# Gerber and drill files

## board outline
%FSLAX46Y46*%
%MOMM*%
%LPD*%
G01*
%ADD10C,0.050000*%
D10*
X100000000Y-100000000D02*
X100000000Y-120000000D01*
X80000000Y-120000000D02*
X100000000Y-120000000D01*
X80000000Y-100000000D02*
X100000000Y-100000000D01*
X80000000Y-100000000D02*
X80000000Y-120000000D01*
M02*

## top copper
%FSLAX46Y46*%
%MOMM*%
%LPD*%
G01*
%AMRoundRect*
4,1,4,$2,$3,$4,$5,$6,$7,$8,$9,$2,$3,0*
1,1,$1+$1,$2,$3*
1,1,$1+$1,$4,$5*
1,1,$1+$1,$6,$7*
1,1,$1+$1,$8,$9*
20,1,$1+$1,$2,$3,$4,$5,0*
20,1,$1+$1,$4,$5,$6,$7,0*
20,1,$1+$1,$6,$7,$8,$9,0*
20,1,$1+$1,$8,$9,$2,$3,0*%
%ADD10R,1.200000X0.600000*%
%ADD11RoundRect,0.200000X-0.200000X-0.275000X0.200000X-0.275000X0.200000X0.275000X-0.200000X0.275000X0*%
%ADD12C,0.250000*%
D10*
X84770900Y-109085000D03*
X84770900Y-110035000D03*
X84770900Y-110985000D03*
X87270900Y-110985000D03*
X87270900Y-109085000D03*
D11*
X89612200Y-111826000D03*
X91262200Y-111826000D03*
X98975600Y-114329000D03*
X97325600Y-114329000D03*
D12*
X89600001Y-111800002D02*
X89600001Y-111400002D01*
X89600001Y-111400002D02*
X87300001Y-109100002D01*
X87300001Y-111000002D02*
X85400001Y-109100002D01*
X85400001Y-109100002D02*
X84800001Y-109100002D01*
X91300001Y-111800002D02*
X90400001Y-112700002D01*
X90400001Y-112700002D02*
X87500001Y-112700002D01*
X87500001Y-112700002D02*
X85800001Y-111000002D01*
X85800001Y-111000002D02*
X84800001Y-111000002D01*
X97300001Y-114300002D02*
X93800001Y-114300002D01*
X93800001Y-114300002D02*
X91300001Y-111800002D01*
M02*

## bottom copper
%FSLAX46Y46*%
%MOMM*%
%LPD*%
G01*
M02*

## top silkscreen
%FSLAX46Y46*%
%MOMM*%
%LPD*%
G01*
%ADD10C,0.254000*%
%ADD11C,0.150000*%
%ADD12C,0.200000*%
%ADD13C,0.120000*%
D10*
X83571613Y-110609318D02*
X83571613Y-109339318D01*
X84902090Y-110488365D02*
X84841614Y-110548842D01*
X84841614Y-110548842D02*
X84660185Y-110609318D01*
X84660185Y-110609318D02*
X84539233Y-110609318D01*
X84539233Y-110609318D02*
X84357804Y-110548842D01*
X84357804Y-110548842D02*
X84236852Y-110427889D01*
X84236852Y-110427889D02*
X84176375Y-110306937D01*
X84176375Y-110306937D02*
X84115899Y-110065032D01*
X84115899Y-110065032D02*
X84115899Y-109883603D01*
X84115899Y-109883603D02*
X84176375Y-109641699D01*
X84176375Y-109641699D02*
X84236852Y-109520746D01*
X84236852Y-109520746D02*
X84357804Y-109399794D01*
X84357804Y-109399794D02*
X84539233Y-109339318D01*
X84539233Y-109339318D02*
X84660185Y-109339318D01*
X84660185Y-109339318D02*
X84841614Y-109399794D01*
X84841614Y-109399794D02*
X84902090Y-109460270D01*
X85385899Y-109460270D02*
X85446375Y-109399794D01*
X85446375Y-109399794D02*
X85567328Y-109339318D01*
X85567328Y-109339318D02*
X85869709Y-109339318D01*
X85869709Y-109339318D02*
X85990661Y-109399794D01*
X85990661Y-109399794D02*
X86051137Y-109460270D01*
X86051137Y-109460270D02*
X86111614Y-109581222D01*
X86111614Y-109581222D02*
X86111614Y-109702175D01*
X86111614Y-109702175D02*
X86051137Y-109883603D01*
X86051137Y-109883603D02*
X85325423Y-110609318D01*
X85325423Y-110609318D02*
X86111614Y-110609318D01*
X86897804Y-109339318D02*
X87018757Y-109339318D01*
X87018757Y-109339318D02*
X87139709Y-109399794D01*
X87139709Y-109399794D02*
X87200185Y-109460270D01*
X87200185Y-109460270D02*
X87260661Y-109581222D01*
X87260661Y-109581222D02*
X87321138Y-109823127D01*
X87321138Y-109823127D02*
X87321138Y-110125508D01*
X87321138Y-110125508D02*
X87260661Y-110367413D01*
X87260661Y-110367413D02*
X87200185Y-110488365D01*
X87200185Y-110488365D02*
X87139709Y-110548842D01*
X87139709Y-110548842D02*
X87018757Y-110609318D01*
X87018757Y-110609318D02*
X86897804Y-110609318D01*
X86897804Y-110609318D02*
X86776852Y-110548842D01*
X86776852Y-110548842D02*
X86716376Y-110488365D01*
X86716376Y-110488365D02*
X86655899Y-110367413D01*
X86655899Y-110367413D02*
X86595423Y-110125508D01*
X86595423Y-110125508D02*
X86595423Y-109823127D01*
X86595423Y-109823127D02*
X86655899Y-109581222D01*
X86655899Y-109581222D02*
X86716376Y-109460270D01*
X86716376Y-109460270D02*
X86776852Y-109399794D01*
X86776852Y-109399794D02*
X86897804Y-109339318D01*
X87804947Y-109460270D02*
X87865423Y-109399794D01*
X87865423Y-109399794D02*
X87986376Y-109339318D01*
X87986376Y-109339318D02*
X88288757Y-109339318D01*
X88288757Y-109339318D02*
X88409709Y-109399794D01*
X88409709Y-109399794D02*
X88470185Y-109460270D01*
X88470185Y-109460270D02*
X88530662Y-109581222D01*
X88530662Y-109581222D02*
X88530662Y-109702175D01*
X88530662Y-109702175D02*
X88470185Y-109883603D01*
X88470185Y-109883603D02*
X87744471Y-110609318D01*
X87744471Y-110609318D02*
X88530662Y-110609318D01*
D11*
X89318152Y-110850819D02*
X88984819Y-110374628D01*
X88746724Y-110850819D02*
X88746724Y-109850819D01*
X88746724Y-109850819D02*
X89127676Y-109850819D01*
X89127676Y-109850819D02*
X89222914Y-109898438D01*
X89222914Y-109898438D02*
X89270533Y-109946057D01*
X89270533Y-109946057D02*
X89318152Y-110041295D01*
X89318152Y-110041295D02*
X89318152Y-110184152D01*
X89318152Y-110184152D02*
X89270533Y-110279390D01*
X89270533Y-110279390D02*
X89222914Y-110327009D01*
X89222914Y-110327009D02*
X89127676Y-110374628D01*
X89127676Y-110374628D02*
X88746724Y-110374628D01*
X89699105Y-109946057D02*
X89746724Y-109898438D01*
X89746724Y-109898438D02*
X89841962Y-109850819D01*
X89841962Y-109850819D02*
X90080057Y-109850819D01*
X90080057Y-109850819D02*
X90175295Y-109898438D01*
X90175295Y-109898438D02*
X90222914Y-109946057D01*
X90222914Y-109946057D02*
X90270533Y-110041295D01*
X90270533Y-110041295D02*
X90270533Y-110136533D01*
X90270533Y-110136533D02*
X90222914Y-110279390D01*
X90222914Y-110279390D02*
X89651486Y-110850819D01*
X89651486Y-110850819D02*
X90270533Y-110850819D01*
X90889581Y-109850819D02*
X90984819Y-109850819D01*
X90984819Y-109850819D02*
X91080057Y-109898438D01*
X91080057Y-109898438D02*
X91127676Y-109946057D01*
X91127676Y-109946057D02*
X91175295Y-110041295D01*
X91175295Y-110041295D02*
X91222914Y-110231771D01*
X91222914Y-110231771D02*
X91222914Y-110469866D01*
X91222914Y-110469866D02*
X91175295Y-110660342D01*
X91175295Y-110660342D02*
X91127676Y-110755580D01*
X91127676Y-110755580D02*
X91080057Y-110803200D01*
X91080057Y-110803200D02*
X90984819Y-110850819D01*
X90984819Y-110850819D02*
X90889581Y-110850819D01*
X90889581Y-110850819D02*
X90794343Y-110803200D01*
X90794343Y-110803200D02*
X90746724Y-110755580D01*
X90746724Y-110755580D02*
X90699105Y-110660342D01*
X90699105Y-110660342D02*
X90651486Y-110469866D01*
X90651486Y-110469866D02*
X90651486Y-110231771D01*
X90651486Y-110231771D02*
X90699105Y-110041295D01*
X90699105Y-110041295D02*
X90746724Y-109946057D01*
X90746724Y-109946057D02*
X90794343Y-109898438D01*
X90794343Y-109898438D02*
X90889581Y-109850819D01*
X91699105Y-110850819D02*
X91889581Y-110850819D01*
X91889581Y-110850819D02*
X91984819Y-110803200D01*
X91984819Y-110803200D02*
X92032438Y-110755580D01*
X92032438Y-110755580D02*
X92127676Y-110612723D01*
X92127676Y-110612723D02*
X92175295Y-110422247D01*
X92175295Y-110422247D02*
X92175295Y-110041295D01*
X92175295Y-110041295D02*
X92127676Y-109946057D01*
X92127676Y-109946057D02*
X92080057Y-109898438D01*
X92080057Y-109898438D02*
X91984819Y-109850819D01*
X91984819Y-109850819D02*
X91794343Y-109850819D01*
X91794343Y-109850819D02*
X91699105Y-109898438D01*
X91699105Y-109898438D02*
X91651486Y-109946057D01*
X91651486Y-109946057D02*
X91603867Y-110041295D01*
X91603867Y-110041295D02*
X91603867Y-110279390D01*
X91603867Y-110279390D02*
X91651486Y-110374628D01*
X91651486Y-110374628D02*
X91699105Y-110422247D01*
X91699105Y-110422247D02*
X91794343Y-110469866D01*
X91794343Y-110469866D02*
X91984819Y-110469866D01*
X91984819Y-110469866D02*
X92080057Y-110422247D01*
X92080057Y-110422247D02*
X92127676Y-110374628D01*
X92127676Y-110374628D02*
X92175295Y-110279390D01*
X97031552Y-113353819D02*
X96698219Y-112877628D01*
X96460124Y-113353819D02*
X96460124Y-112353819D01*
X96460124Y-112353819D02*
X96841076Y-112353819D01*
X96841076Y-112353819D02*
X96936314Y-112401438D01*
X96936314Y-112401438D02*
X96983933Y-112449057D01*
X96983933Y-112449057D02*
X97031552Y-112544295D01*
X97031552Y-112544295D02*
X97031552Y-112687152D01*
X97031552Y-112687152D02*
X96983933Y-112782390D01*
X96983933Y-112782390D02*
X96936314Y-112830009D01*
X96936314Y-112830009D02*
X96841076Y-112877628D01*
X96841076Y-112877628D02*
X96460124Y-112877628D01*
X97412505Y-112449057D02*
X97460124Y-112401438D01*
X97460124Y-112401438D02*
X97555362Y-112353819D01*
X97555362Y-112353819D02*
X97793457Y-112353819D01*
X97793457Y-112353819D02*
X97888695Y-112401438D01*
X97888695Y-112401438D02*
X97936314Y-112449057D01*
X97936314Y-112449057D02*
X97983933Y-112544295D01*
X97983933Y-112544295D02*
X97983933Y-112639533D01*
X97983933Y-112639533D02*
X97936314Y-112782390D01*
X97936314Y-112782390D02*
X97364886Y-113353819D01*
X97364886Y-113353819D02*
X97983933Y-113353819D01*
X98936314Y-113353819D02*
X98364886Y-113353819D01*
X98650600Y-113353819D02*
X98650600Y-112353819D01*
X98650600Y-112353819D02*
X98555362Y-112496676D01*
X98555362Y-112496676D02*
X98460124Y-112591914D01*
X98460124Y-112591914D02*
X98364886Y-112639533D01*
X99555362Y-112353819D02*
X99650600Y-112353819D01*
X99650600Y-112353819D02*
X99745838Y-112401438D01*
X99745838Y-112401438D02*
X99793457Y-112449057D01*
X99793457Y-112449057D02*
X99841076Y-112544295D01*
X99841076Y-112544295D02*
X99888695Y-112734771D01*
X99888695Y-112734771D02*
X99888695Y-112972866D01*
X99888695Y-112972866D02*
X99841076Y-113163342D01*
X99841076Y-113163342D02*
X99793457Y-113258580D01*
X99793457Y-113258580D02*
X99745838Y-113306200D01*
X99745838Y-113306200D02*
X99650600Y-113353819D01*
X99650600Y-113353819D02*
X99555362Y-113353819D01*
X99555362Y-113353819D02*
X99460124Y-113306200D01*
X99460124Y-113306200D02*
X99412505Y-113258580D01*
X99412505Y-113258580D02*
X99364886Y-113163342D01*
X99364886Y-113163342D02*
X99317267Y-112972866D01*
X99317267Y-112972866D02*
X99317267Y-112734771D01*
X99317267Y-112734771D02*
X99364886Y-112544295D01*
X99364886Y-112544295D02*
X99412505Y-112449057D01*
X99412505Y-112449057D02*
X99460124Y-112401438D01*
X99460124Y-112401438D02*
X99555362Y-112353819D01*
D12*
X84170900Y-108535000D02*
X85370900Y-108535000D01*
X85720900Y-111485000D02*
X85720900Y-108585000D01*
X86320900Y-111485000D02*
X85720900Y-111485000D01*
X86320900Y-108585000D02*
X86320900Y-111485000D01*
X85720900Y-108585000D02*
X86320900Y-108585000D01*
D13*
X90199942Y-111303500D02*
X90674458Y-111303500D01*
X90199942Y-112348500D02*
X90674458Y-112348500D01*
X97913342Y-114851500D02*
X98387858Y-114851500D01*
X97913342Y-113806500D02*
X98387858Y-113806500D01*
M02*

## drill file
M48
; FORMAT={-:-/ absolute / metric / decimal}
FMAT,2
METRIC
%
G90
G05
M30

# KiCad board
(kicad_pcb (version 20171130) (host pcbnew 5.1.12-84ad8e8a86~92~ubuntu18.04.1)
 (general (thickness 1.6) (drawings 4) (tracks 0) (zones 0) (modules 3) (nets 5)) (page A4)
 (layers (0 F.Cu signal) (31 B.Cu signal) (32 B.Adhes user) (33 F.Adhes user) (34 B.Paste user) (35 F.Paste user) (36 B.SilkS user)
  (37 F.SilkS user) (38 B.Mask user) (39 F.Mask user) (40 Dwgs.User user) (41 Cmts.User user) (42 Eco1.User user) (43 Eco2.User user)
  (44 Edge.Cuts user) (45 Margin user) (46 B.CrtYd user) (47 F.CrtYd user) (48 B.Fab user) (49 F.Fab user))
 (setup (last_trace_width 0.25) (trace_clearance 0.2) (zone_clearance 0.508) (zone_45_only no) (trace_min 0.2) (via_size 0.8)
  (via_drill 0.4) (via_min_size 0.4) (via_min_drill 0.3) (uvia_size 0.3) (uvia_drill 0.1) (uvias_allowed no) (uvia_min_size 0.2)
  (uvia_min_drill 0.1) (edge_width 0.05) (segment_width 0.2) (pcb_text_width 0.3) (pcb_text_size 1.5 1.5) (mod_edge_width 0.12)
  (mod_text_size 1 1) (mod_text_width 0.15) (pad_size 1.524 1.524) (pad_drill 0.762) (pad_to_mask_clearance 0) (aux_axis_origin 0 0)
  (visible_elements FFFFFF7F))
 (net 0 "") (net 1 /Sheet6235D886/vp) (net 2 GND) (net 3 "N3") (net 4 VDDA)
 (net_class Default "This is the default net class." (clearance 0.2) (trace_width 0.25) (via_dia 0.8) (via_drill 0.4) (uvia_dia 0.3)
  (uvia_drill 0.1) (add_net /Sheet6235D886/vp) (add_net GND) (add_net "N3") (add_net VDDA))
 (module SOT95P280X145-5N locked (layer F.Cu) (at 86.020900 110.035000)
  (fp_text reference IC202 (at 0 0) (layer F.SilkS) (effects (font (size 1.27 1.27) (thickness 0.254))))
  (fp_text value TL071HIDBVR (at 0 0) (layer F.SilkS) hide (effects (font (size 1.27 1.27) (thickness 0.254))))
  (fp_line (start -1.85 -1.5) (end -0.65 -1.5) (layer F.SilkS) (width 0.2))
  (fp_line (start -0.3 1.45) (end -0.3 -1.45) (layer F.SilkS) (width 0.2))
  (fp_line (start 0.3 1.45) (end -0.3 1.45) (layer F.SilkS) (width 0.2))
  (fp_line (start 0.3 -1.45) (end 0.3 1.45) (layer F.SilkS) (width 0.2))
  (fp_line (start -0.3 -1.45) (end 0.3 -1.45) (layer F.SilkS) (width 0.2))
  (pad 1 smd rect (at -1.25 -0.95 90.000000) (size 0.6 1.2) (layers F.Cu F.Mask F.Paste) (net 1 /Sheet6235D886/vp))
  (pad 2 smd rect (at -1.25 0 90.000000) (size 0.6 1.2) (layers F.Cu F.Mask F.Paste) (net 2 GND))
  (pad 3 smd rect (at -1.25 0.95 90.000000) (size 0.6 1.2) (layers F.Cu F.Mask F.Paste) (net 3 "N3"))
  (pad 4 smd rect (at 1.25 0.95 90.000000) (size 0.6 1.2) (layers F.Cu F.Mask F.Paste) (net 1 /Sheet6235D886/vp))
  (pad 5 smd rect (at 1.25 -0.95 90.000000) (size 0.6 1.2) (layers F.Cu F.Mask F.Paste) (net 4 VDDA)))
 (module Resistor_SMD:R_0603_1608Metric (layer F.Cu) (at 90.437200 111.826000)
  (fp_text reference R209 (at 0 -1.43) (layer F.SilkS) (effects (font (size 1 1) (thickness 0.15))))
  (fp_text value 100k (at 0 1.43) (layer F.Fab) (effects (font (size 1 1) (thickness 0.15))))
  (fp_line (start -0.237258 -0.5225) (end 0.237258 -0.5225) (layer F.SilkS) (width 0.12))
  (fp_line (start -0.237258 0.5225) (end 0.237258 0.5225) (layer F.SilkS) (width 0.12))
  (pad 1 smd roundrect (at -0.825 0) (size 0.8 0.95) (layers F.Cu F.Mask F.Paste) (roundrect_rratio 0.25) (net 4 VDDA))
  (pad 2 smd roundrect (at 0.825 0) (size 0.8 0.95) (layers F.Cu F.Mask F.Paste) (roundrect_rratio 0.25) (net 3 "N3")))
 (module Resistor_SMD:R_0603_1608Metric (layer F.Cu) (at 98.150600 114.329000)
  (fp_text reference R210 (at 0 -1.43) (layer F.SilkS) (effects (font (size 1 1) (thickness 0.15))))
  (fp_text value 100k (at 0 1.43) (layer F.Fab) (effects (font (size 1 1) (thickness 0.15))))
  (fp_line (start -0.237258 0.5225) (end 0.237258 0.5225) (layer F.SilkS) (width 0.12))
  (fp_line (start -0.237258 -0.5225) (end 0.237258 -0.5225) (layer F.SilkS) (width 0.12))
  (pad 2 smd roundrect (at 0.825 0) (size 0.8 0.95) (layers F.Cu F.Mask F.Paste) (roundrect_rratio 0.25) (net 2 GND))
  (pad 1 smd roundrect (at -0.825 0) (size 0.8 0.95) (layers F.Cu F.Mask F.Paste) (roundrect_rratio 0.25) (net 3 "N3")))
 (gr_line (start 100 100) (end 100 120) (layer Edge.Cuts) (width 0.05))
 (gr_line (start 80 120) (end 100 120) (layer Edge.Cuts) (width 0.05))
 (gr_line (start 80 100) (end 100 100) (layer Edge.Cuts) (width 0.05))
 (gr_line (start 80 100) (end 80 120) (layer Edge.Cuts) (width 0.05))
 (segment (start 89.600001 111.800002) (end 89.600001 111.400002) (width 0.250000) (layer F.Cu) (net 4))
 (segment (start 89.600001 111.400002) (end 87.300001 109.100002) (width 0.250000) (layer F.Cu) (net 4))
 (segment (start 87.300001 111.000002) (end 85.400001 109.100002) (width 0.250000) (layer F.Cu) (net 1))
 (segment (start 85.400001 109.100002) (end 84.800001 109.100002) (width 0.250000) (layer F.Cu) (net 1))
 (segment (start 91.300001 111.800002) (end 90.400001 112.700002) (width 0.250000) (layer F.Cu) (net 3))
 (segment (start 90.400001 112.700002) (end 87.500001 112.700002) (width 0.250000) (layer F.Cu) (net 3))
 (segment (start 87.500001 112.700002) (end 85.800001 111.000002) (width 0.250000) (layer F.Cu) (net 3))
 (segment (start 85.800001 111.000002) (end 84.800001 111.000002) (width 0.250000) (layer F.Cu) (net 3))
 (segment (start 97.300001 114.300002) (end 93.800001 114.300002) (width 0.250000) (layer F.Cu) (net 3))
 (segment (start 93.800001 114.300002) (end 91.300001 111.800002) (width 0.250000) (layer F.Cu) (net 3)))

